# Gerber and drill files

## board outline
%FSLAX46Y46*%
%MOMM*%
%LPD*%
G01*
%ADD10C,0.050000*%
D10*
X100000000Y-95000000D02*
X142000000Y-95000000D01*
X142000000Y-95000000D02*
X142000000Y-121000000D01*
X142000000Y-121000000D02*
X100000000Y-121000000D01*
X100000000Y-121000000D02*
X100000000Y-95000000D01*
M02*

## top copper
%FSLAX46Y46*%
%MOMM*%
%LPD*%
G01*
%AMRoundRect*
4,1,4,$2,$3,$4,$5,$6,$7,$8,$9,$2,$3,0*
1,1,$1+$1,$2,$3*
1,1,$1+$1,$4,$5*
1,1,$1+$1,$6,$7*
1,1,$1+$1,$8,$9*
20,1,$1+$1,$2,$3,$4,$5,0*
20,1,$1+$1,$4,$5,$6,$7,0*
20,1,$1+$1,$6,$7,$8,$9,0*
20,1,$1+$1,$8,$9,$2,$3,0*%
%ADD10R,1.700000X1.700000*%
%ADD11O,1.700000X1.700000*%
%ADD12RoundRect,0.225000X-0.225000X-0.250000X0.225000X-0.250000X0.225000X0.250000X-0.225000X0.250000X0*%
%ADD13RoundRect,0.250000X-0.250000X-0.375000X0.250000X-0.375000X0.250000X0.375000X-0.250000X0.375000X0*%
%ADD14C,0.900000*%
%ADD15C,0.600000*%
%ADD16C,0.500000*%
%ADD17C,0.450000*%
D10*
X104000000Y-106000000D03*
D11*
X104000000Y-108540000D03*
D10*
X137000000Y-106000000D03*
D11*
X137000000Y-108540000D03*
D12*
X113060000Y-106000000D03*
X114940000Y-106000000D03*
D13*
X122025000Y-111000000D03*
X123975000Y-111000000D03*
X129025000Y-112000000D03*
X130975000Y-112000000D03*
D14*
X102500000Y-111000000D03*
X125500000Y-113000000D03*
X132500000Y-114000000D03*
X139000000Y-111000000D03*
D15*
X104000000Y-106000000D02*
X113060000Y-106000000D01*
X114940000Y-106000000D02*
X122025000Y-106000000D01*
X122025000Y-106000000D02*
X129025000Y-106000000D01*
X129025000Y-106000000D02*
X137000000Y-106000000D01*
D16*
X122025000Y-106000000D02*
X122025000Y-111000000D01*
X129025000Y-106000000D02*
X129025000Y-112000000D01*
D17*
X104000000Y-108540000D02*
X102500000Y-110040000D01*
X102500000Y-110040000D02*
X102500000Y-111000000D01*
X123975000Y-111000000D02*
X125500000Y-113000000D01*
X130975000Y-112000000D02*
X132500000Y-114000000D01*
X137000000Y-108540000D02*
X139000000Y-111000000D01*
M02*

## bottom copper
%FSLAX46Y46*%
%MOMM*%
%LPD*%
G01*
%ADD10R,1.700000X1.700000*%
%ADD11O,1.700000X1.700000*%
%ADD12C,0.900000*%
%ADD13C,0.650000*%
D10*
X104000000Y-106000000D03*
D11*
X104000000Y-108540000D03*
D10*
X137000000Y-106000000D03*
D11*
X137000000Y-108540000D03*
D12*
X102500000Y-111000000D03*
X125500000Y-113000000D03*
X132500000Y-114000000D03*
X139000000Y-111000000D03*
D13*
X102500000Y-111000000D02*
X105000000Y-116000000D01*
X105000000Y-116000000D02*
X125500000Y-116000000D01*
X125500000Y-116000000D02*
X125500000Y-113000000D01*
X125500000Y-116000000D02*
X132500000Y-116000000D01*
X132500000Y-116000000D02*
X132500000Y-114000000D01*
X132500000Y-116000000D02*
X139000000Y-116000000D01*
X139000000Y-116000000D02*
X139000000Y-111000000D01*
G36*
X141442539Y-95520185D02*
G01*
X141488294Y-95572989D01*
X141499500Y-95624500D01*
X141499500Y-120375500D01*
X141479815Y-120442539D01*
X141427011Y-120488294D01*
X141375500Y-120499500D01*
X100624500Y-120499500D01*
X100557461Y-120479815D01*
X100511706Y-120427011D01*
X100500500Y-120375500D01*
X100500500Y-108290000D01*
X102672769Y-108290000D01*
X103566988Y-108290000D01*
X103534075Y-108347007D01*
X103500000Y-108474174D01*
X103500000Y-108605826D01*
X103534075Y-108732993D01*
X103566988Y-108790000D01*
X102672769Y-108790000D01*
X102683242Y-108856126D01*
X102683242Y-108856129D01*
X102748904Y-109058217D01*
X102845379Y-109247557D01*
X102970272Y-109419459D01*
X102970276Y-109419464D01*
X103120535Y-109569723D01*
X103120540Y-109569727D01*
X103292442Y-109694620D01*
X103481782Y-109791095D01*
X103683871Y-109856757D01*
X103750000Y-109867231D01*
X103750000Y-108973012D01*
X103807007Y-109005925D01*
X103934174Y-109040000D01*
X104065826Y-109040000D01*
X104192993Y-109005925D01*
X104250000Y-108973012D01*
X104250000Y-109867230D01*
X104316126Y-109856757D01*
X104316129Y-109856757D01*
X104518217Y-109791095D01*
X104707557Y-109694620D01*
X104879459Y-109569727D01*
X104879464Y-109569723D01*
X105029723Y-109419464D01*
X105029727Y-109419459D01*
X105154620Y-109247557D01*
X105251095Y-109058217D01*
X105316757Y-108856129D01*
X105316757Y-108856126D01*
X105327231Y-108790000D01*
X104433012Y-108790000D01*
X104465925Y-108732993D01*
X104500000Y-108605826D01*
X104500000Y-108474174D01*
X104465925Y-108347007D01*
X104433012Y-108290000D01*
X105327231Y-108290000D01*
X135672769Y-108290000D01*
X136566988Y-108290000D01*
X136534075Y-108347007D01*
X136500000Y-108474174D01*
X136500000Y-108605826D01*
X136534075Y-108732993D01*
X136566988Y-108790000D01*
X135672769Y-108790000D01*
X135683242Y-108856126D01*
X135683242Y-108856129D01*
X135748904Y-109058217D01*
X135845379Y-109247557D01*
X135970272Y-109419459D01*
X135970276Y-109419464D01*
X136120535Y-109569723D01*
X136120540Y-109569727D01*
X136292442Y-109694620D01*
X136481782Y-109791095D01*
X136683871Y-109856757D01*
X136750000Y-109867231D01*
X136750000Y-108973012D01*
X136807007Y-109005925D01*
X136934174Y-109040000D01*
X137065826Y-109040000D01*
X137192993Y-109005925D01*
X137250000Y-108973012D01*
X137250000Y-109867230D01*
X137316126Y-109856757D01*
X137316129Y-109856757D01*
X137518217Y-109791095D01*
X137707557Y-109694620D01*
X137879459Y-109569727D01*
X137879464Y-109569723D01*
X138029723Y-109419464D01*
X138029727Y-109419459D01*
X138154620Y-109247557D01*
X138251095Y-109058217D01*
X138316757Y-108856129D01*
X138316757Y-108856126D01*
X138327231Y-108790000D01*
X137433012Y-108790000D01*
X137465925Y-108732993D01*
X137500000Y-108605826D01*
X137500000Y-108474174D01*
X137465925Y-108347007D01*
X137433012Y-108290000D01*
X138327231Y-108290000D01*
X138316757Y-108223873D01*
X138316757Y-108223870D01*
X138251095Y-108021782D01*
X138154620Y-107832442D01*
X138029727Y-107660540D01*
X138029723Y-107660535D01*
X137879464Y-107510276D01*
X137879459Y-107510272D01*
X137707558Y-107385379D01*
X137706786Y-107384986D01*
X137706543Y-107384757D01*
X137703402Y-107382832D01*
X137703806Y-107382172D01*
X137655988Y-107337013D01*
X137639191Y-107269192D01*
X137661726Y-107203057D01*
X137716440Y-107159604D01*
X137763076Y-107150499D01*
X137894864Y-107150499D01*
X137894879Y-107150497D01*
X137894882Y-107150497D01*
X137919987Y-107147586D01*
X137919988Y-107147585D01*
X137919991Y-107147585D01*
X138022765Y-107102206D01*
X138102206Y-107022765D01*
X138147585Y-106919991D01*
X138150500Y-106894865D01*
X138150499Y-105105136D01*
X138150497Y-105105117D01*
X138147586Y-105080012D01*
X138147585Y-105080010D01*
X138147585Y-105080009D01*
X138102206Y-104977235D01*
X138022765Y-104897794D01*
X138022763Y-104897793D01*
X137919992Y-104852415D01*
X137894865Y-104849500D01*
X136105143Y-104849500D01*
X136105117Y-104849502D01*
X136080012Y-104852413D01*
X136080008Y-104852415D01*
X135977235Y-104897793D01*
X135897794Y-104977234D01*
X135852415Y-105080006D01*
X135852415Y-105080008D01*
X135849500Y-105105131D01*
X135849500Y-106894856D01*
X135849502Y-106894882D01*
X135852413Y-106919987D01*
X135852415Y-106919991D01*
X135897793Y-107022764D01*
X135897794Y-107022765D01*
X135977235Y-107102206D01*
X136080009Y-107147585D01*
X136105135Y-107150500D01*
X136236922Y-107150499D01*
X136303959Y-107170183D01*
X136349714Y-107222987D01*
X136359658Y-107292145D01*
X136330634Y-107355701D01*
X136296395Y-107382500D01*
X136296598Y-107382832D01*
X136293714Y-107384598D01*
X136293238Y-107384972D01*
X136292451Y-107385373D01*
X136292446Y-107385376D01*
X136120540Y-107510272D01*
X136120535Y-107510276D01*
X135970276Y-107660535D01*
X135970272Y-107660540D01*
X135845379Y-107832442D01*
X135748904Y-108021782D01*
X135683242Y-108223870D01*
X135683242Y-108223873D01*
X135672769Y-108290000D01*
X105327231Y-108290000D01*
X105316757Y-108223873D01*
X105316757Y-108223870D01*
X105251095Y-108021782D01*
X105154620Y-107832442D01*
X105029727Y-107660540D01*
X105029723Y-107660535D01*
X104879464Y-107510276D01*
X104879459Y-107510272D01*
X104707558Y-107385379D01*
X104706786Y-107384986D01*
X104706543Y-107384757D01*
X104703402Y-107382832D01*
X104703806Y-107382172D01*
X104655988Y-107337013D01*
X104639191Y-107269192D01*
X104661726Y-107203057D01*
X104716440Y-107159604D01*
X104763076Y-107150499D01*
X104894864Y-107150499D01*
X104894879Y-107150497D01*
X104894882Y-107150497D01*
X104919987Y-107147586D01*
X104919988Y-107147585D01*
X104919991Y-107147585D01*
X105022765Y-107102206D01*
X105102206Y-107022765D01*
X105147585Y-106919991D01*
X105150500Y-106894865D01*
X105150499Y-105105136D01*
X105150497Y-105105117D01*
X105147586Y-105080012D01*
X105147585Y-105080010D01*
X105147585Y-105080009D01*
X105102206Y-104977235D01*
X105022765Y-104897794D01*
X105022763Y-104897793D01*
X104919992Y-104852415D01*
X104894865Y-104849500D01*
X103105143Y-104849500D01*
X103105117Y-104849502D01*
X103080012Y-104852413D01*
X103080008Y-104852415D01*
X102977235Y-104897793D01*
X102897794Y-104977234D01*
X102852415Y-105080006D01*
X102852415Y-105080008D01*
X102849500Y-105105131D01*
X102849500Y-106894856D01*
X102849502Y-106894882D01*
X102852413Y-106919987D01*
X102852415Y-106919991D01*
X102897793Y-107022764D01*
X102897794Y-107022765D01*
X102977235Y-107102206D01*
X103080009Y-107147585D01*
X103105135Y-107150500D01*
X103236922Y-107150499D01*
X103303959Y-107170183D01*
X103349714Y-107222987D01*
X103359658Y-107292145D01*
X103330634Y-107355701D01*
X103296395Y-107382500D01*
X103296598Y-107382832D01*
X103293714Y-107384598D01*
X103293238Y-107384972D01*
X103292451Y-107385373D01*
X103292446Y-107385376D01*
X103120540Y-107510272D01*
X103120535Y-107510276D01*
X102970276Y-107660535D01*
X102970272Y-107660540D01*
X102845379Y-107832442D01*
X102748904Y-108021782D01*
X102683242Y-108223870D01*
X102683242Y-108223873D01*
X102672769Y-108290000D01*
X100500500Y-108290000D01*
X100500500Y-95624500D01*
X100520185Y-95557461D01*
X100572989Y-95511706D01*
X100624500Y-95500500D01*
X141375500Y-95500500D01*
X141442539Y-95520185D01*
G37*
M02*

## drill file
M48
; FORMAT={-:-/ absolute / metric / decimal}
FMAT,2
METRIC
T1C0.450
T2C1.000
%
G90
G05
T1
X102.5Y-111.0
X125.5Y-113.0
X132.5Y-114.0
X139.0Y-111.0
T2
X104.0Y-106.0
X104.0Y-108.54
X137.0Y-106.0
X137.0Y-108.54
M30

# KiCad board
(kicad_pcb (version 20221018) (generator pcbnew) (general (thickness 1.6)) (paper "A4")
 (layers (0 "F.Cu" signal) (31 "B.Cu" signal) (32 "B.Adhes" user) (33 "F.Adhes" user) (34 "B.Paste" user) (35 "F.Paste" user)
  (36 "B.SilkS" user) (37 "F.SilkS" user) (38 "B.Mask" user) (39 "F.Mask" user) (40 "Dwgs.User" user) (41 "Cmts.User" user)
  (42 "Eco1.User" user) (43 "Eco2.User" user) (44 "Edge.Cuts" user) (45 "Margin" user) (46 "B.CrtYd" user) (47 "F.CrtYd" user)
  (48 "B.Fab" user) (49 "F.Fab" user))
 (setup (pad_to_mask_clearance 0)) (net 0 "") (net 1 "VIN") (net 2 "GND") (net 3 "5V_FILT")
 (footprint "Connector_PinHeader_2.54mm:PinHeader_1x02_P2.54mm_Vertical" (layer "F.Cu") (at 104 106)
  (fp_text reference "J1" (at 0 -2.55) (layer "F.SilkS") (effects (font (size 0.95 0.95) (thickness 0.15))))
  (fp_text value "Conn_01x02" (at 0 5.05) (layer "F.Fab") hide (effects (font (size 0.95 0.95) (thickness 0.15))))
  (pad "1" thru_hole rect (at 0 0 0) (size 1.7 1.7) (drill 1) (layers "*.Cu" "*.Mask") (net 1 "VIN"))
  (pad "2" thru_hole oval (at 0 2.54 0) (size 1.7 1.7) (drill 1) (layers "*.Cu" "*.Mask") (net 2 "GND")))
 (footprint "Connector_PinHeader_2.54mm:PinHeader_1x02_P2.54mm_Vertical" (layer "F.Cu") (at 137 106)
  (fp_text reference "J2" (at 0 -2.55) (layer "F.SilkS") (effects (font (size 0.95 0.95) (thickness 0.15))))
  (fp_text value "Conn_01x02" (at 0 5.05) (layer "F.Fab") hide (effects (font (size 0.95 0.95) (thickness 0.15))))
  (pad "1" thru_hole rect (at 0 0 0) (size 1.7 1.7) (drill 1) (layers "*.Cu" "*.Mask") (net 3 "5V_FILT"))
  (pad "2" thru_hole oval (at 0 2.54 0) (size 1.7 1.7) (drill 1) (layers "*.Cu" "*.Mask") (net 2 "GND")))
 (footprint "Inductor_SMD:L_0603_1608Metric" (layer "F.Cu") (at 114 106)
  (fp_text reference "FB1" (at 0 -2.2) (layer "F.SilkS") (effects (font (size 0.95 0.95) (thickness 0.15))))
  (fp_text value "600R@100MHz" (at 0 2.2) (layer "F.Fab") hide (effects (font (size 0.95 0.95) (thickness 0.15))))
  (pad "1" smd roundrect (at -0.94 0 0) (size 0.9 0.95) (layers "F.Cu" "F.Paste" "F.Mask") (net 1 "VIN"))
  (pad "2" smd roundrect (at 0.94 0 0) (size 0.9 0.95) (layers "F.Cu" "F.Paste" "F.Mask") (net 3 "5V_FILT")))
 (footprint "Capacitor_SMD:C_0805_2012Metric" (layer "F.Cu") (at 123 111)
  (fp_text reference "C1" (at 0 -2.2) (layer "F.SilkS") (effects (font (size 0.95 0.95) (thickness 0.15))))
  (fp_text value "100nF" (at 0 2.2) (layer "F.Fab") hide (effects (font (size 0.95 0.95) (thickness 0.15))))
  (pad "1" smd roundrect (at -0.975 0 0) (size 1.0 1.25) (layers "F.Cu" "F.Paste" "F.Mask") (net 3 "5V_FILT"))
  (pad "2" smd roundrect (at 0.975 0 0) (size 1.0 1.25) (layers "F.Cu" "F.Paste" "F.Mask") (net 2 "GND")))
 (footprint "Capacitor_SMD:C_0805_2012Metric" (layer "F.Cu") (at 130 112)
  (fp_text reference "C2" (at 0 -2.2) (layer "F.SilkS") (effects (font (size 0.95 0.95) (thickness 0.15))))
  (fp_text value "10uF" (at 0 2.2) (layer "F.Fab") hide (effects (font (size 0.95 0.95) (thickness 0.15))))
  (pad "1" smd roundrect (at -0.975 0 0) (size 1.0 1.25) (layers "F.Cu" "F.Paste" "F.Mask") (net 3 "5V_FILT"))
  (pad "2" smd roundrect (at 0.975 0 0) (size 1.0 1.25) (layers "F.Cu" "F.Paste" "F.Mask") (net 2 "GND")))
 (segment (start 104 106) (end 113.06 106) (width 0.6) (layer "F.Cu") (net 1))
 (segment (start 114.94 106) (end 122.025 106) (width 0.6) (layer "F.Cu") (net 3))
 (segment (start 122.025 106) (end 129.025 106) (width 0.6) (layer "F.Cu") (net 3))
 (segment (start 129.025 106) (end 137 106) (width 0.6) (layer "F.Cu") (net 3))
 (segment (start 122.025 106) (end 122.025 111) (width 0.5) (layer "F.Cu") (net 3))
 (segment (start 129.025 106) (end 129.025 112) (width 0.5) (layer "F.Cu") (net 3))
 (segment (start 104 108.54) (end 102.5 110.04) (width 0.45) (layer "F.Cu") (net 2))
 (segment (start 102.5 110.04) (end 102.5 111) (width 0.45) (layer "F.Cu") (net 2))
 (segment (start 123.975 111) (end 125.5 113) (width 0.45) (layer "F.Cu") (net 2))
 (segment (start 130.975 112) (end 132.5 114) (width 0.45) (layer "F.Cu") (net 2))
 (segment (start 137 108.54) (end 139 111) (width 0.45) (layer "F.Cu") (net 2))
 (segment (start 102.5 111) (end 105 116) (width 0.65) (layer "B.Cu") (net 2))
 (segment (start 105 116) (end 125.5 116) (width 0.65) (layer "B.Cu") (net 2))
 (segment (start 125.5 116) (end 125.5 113) (width 0.65) (layer "B.Cu") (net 2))
 (segment (start 125.5 116) (end 132.5 116) (width 0.65) (layer "B.Cu") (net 2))
 (segment (start 132.5 116) (end 132.5 114) (width 0.65) (layer "B.Cu") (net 2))
 (segment (start 132.5 116) (end 139 116) (width 0.65) (layer "B.Cu") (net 2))
 (segment (start 139 116) (end 139 111) (width 0.65) (layer "B.Cu") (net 2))
 (via (at 102.5 111) (size 0.9) (drill 0.45) (layers "F.Cu" "B.Cu") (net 2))
 (via (at 125.5 113) (size 0.9) (drill 0.45) (layers "F.Cu" "B.Cu") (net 2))
 (via (at 132.5 114) (size 0.9) (drill 0.45) (layers "F.Cu" "B.Cu") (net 2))
 (via (at 139 111) (size 0.9) (drill 0.45) (layers "F.Cu" "B.Cu") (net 2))
 (gr_line (start 100 95) (end 142 95) (stroke (width 0.05) (type default)) (layer "Edge.Cuts"))
 (gr_line (start 142 95) (end 142 121) (stroke (width 0.05) (type default)) (layer "Edge.Cuts"))
 (gr_line (start 142 121) (end 100 121) (stroke (width 0.05) (type default)) (layer "Edge.Cuts"))
 (gr_line (start 100 121) (end 100 95) (stroke (width 0.05) (type default)) (layer "Edge.Cuts"))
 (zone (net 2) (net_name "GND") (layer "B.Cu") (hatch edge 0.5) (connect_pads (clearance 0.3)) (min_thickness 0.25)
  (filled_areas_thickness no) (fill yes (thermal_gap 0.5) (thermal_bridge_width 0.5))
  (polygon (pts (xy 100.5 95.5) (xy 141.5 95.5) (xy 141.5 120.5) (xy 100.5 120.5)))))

